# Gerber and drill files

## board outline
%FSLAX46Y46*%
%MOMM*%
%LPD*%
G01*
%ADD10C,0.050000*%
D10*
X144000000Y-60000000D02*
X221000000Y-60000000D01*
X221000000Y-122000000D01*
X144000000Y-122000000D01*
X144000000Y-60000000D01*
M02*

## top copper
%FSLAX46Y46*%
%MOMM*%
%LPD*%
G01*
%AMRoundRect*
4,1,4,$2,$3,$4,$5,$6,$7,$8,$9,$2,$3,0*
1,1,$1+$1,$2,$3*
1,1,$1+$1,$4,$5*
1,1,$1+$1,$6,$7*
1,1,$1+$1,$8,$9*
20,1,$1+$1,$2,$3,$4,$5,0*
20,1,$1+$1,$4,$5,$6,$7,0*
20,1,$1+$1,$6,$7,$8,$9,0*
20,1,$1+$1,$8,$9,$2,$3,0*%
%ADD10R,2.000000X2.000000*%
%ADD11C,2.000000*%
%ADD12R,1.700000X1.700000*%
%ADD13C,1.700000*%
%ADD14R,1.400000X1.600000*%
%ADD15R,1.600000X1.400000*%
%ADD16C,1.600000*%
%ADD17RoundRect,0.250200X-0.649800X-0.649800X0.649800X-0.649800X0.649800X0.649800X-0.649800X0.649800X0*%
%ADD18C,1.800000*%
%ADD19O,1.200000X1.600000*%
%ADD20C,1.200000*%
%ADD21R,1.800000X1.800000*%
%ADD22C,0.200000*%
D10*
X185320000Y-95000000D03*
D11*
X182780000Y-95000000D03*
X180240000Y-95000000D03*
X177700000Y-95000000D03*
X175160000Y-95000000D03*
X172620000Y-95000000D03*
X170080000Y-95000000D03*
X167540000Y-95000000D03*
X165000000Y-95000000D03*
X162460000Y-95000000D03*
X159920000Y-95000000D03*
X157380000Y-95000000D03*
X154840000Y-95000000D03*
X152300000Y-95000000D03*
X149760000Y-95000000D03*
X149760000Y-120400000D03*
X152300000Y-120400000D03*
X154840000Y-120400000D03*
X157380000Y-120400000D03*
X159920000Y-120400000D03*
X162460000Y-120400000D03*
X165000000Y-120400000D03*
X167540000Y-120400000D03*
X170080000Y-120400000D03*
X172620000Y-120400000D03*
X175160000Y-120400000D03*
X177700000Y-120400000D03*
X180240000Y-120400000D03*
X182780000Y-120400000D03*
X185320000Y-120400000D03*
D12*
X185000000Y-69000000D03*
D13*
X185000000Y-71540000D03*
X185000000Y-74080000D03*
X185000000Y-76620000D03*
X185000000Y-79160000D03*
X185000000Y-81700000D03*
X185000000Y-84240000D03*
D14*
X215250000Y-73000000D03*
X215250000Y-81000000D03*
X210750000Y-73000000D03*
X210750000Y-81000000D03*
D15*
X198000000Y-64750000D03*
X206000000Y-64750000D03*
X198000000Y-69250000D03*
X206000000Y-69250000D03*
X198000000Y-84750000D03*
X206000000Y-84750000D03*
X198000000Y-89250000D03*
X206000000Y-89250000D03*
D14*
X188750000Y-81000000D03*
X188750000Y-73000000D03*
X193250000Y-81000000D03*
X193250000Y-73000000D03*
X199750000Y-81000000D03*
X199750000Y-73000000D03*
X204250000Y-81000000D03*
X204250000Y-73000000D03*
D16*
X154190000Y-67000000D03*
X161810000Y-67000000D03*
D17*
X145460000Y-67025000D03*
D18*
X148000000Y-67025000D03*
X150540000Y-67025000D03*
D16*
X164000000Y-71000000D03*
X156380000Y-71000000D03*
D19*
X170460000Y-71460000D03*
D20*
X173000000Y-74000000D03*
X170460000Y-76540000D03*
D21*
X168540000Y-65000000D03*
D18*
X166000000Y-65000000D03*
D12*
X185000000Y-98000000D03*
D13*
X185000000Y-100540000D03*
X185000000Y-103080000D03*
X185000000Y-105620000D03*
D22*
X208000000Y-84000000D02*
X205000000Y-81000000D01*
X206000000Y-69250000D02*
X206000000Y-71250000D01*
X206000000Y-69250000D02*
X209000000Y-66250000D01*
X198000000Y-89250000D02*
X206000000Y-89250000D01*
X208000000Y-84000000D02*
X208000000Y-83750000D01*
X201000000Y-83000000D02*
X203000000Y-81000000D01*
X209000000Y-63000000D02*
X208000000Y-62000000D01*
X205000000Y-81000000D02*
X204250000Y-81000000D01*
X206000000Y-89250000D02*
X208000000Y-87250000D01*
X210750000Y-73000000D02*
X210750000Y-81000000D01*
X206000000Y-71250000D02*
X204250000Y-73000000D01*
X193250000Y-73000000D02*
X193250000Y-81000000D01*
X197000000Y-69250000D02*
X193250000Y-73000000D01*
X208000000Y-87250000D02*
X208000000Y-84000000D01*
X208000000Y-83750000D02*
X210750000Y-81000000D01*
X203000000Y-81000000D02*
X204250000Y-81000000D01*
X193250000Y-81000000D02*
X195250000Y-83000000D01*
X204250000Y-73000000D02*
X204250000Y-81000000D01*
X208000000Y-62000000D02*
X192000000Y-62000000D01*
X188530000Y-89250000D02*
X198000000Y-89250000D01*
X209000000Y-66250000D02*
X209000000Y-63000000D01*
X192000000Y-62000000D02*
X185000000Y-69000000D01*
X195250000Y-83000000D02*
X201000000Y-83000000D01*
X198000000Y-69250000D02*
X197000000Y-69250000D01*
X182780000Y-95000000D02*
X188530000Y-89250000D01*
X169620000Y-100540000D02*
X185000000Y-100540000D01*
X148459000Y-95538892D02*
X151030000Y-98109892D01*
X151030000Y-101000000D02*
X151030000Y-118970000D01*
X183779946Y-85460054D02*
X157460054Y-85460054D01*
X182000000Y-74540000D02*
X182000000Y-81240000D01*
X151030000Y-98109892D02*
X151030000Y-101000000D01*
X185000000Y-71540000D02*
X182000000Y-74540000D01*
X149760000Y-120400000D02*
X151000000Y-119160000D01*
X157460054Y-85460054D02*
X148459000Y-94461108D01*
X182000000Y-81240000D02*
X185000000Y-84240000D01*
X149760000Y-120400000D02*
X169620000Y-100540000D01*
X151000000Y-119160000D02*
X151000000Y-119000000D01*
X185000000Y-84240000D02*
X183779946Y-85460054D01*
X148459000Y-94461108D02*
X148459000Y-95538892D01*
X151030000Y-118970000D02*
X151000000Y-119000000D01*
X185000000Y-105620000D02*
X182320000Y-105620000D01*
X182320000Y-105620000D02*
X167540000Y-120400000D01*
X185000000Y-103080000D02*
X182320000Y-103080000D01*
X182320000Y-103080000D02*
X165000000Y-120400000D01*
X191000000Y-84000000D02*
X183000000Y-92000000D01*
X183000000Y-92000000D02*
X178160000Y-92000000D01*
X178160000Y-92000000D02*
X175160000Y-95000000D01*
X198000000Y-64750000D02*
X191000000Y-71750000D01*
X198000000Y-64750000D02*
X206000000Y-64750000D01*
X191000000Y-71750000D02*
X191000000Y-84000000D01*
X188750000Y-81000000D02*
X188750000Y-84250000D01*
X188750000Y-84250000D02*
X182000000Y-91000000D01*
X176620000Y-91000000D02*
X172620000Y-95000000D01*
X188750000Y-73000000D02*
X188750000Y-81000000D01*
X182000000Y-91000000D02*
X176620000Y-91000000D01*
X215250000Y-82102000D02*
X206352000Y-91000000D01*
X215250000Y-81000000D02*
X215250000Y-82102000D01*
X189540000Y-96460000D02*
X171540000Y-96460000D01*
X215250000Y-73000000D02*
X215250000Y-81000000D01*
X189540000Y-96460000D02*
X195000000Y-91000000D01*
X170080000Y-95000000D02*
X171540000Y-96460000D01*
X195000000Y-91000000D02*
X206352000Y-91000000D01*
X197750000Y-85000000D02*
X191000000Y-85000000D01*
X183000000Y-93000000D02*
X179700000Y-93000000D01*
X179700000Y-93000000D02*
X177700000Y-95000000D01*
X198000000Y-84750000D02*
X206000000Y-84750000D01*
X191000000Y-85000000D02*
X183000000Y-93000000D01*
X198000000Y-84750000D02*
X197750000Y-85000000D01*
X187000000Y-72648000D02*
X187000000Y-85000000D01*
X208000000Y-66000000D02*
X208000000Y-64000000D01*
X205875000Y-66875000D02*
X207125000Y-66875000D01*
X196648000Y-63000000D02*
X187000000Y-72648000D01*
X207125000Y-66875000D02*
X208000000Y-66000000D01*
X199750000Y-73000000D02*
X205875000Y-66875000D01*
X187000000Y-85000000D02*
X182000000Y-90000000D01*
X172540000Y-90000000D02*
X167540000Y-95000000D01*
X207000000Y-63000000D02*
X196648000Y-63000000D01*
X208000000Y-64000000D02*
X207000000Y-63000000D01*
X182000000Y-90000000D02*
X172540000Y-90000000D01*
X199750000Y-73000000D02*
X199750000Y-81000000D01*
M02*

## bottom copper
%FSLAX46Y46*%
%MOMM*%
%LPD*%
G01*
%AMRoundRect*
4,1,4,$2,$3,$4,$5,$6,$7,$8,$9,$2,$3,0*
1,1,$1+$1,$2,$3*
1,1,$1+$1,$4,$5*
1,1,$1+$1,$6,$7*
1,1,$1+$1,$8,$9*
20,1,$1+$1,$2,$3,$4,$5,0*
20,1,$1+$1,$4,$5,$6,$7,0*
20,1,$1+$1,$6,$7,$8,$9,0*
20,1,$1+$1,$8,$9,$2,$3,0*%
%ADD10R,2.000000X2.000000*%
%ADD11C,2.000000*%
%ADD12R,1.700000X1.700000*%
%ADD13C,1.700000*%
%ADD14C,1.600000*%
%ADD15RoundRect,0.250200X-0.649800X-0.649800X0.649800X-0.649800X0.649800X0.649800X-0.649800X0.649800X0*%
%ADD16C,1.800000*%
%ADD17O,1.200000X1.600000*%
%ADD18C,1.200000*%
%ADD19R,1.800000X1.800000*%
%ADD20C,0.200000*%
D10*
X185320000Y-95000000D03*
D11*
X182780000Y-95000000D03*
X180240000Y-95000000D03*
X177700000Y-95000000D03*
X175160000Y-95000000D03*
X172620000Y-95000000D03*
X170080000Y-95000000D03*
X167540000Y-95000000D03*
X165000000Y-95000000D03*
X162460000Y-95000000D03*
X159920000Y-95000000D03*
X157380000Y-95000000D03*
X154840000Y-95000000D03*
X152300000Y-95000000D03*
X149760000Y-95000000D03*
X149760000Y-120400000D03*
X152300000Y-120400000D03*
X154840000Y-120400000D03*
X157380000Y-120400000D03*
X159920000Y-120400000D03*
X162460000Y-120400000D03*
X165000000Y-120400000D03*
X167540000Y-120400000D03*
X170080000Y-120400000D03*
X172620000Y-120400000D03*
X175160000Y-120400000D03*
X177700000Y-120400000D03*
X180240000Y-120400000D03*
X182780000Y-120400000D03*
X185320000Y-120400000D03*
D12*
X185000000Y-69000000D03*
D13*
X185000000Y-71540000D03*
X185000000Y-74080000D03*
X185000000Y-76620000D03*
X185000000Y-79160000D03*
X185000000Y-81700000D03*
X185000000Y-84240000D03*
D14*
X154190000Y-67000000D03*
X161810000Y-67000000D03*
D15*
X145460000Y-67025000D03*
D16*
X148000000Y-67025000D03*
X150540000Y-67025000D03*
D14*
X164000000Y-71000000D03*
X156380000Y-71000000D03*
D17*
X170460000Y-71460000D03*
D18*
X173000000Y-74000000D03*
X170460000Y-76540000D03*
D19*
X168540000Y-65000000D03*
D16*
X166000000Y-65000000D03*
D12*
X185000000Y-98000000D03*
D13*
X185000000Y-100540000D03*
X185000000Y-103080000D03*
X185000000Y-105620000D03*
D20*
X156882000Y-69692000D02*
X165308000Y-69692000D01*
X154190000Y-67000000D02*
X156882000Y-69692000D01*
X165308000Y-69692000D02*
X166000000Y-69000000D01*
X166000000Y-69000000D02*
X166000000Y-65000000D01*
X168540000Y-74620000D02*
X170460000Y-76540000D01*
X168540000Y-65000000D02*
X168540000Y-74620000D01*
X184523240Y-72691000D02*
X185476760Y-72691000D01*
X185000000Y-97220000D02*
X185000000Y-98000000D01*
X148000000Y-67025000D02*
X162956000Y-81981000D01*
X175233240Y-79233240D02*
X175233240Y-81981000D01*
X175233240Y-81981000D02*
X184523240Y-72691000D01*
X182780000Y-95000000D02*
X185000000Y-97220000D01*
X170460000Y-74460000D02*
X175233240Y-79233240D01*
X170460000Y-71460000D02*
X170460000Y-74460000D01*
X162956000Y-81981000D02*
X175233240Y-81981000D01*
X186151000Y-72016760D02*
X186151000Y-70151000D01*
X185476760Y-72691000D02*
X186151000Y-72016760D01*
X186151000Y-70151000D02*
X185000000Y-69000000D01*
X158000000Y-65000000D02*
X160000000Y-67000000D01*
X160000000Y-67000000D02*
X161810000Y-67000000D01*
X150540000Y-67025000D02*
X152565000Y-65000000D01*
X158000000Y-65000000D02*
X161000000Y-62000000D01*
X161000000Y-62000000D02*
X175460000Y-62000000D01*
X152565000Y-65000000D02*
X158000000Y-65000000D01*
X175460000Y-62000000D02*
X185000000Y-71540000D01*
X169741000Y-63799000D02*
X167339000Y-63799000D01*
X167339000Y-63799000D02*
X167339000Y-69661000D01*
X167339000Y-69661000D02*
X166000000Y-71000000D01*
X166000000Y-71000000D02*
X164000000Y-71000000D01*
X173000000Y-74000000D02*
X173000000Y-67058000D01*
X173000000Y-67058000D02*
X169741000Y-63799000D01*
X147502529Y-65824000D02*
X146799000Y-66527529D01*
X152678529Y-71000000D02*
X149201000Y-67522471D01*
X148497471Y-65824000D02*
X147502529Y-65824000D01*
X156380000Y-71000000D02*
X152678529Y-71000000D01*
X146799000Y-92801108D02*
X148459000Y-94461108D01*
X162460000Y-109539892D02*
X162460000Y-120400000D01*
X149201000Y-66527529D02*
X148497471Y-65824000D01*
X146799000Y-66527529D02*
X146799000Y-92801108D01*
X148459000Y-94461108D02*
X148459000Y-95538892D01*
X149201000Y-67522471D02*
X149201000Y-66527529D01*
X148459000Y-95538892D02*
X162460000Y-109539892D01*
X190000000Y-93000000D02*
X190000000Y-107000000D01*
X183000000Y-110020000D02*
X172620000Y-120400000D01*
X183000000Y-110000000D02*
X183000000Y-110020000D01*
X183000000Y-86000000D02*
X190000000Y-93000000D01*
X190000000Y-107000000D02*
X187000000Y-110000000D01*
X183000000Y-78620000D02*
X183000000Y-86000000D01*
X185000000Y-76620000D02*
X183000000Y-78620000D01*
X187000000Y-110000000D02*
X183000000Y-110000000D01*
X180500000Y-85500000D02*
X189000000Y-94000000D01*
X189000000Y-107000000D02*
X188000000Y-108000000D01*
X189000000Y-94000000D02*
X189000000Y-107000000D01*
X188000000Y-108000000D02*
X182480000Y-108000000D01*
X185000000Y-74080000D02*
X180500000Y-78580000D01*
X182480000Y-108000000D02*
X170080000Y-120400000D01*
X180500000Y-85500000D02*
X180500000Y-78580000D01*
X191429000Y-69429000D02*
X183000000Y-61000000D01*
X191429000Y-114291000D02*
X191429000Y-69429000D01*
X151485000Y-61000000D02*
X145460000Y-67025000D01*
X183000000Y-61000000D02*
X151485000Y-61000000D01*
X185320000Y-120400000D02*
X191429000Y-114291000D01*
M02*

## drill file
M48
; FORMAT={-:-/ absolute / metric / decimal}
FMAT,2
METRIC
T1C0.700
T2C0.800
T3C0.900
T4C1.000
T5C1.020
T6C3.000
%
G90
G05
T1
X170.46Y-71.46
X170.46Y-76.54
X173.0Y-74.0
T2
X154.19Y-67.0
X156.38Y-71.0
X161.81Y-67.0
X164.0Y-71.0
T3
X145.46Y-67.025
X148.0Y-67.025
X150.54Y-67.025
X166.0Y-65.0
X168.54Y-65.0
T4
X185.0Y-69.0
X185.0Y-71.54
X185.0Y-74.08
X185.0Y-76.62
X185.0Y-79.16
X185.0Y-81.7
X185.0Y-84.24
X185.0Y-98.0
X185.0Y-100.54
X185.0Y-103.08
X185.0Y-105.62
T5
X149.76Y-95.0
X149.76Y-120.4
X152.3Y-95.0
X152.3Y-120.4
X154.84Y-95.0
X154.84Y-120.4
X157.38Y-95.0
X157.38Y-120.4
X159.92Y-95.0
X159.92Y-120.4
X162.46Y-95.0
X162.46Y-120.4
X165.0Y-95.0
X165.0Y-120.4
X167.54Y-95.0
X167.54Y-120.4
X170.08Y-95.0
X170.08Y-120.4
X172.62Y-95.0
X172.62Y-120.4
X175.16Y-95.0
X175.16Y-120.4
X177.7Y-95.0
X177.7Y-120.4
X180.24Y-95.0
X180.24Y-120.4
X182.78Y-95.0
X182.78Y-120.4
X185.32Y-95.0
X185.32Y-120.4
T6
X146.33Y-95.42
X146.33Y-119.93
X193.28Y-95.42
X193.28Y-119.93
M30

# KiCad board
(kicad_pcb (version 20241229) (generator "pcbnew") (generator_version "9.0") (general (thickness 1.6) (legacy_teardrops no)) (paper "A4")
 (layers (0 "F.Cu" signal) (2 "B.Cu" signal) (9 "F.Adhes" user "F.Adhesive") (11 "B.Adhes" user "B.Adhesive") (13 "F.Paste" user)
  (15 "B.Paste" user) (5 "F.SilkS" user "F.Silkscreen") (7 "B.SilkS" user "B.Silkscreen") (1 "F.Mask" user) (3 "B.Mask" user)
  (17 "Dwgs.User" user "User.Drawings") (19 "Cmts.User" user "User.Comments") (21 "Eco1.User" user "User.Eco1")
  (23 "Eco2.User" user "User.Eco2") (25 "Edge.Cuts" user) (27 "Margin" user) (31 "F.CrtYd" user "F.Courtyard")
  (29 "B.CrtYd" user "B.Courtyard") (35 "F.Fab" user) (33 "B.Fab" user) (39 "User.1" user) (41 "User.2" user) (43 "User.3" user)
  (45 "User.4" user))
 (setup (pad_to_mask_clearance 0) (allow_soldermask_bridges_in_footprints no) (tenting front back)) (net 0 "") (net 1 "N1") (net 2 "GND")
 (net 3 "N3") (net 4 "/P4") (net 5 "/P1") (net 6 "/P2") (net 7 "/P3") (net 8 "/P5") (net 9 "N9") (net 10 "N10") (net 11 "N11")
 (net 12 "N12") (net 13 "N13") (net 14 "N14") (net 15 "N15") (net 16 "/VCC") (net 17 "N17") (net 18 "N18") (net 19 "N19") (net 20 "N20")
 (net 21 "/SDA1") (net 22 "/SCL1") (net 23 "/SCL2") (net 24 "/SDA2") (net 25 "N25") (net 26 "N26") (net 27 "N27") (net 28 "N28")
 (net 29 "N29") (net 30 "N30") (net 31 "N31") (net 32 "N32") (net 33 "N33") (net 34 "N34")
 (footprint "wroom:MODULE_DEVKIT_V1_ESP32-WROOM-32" (layer "F.Cu") (at 169.805 107.7 -90)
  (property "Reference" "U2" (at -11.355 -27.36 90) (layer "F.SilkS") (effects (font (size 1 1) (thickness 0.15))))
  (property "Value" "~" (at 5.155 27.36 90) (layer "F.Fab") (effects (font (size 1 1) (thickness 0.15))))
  (pad "" np_thru_hole circle (at -12.28 -23.475 270) (size 3 3) (drill 3) (layers "*.Cu" "*.Mask"))
  (pad "" np_thru_hole circle (at -12.28 23.475 270) (size 3 3) (drill 3) (layers "*.Cu" "*.Mask"))
  (pad "" np_thru_hole circle (at 12.23 -23.475 270) (size 3 3) (drill 3) (layers "*.Cu" "*.Mask"))
  (pad "" np_thru_hole circle (at 12.23 23.475 270) (size 3 3) (drill 3) (layers "*.Cu" "*.Mask"))
  (pad "1" thru_hole rect (at -12.7 -15.515 270) (size 2 2) (drill 1.02) (layers "*.Cu" "*.Mask") (remove_unused_layers no) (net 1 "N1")
   (solder_mask_margin 0.102))
  (pad "2" thru_hole circle (at -12.7 -12.975 270) (size 2 2) (drill 1.02) (layers "*.Cu" "*.Mask") (remove_unused_layers no) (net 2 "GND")
   (solder_mask_margin 0.102))
  (pad "3" thru_hole circle (at -12.7 -10.435 270) (size 2 2) (drill 1.02) (layers "*.Cu" "*.Mask") (remove_unused_layers no) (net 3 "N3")
   (solder_mask_margin 0.102))
  (pad "4" thru_hole circle (at -12.7 -7.895 270) (size 2 2) (drill 1.02) (layers "*.Cu" "*.Mask") (remove_unused_layers no) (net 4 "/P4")
   (solder_mask_margin 0.102))
  (pad "5" thru_hole circle (at -12.7 -5.355 270) (size 2 2) (drill 1.02) (layers "*.Cu" "*.Mask") (remove_unused_layers no) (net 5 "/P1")
   (solder_mask_margin 0.102))
  (pad "6" thru_hole circle (at -12.7 -2.815 270) (size 2 2) (drill 1.02) (layers "*.Cu" "*.Mask") (remove_unused_layers no) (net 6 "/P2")
   (solder_mask_margin 0.102))
  (pad "7" thru_hole circle (at -12.7 -0.275 270) (size 2 2) (drill 1.02) (layers "*.Cu" "*.Mask") (remove_unused_layers no) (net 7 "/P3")
   (solder_mask_margin 0.102))
  (pad "8" thru_hole circle (at -12.7 2.265 270) (size 2 2) (drill 1.02) (layers "*.Cu" "*.Mask") (remove_unused_layers no) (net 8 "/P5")
   (solder_mask_margin 0.102))
  (pad "9" thru_hole circle (at -12.7 4.805 270) (size 2 2) (drill 1.02) (layers "*.Cu" "*.Mask") (remove_unused_layers no) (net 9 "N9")
   (solder_mask_margin 0.102))
  (pad "10" thru_hole circle (at -12.7 7.345 270) (size 2 2) (drill 1.02) (layers "*.Cu" "*.Mask") (remove_unused_layers no) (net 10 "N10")
   (solder_mask_margin 0.102))
  (pad "11" thru_hole circle (at -12.7 9.885 270) (size 2 2) (drill 1.02) (layers "*.Cu" "*.Mask") (remove_unused_layers no) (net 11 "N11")
   (solder_mask_margin 0.102))
  (pad "12" thru_hole circle (at -12.7 12.425 270) (size 2 2) (drill 1.02) (layers "*.Cu" "*.Mask") (remove_unused_layers no) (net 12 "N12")
   (solder_mask_margin 0.102))
  (pad "13" thru_hole circle (at -12.7 14.965 270) (size 2 2) (drill 1.02) (layers "*.Cu" "*.Mask") (remove_unused_layers no) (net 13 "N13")
   (solder_mask_margin 0.102))
  (pad "14" thru_hole circle (at -12.7 17.505 270) (size 2 2) (drill 1.02) (layers "*.Cu" "*.Mask") (remove_unused_layers no) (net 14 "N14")
   (solder_mask_margin 0.102))
  (pad "15" thru_hole circle (at -12.7 20.045 270) (size 2 2) (drill 1.02) (layers "*.Cu" "*.Mask") (remove_unused_layers no) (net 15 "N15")
   (solder_mask_margin 0.102))
  (pad "16" thru_hole circle (at 12.7 20.045 270) (size 2 2) (drill 1.02) (layers "*.Cu" "*.Mask") (remove_unused_layers no) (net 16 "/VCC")
   (solder_mask_margin 0.102))
  (pad "17" thru_hole circle (at 12.7 17.505 270) (size 2 2) (drill 1.02) (layers "*.Cu" "*.Mask") (remove_unused_layers no) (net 2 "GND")
   (solder_mask_margin 0.102))
  (pad "18" thru_hole circle (at 12.7 14.965 270) (size 2 2) (drill 1.02) (layers "*.Cu" "*.Mask") (remove_unused_layers no) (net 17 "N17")
   (solder_mask_margin 0.102))
  (pad "19" thru_hole circle (at 12.7 12.425 270) (size 2 2) (drill 1.02) (layers "*.Cu" "*.Mask") (remove_unused_layers no) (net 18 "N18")
   (solder_mask_margin 0.102))
  (pad "20" thru_hole circle (at 12.7 9.885 270) (size 2 2) (drill 1.02) (layers "*.Cu" "*.Mask") (remove_unused_layers no) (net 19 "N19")
   (solder_mask_margin 0.102))
  (pad "21" thru_hole circle (at 12.7 7.345 270) (size 2 2) (drill 1.02) (layers "*.Cu" "*.Mask") (remove_unused_layers no) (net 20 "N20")
   (solder_mask_margin 0.102))
  (pad "22" thru_hole circle (at 12.7 4.805 270) (size 2 2) (drill 1.02) (layers "*.Cu" "*.Mask") (remove_unused_layers no) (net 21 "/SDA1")
   (solder_mask_margin 0.102))
  (pad "23" thru_hole circle (at 12.7 2.265 270) (size 2 2) (drill 1.02) (layers "*.Cu" "*.Mask") (remove_unused_layers no) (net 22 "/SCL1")
   (solder_mask_margin 0.102))
  (pad "24" thru_hole circle (at 12.7 -0.275 270) (size 2 2) (drill 1.02) (layers "*.Cu" "*.Mask") (remove_unused_layers no)
   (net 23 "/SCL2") (solder_mask_margin 0.102))
  (pad "25" thru_hole circle (at 12.7 -2.815 270) (size 2 2) (drill 1.02) (layers "*.Cu" "*.Mask") (remove_unused_layers no)
   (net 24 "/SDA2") (solder_mask_margin 0.102))
  (pad "26" thru_hole circle (at 12.7 -5.355 270) (size 2 2) (drill 1.02) (layers "*.Cu" "*.Mask") (remove_unused_layers no) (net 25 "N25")
   (solder_mask_margin 0.102))
  (pad "27" thru_hole circle (at 12.7 -7.895 270) (size 2 2) (drill 1.02) (layers "*.Cu" "*.Mask") (remove_unused_layers no) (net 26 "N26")
   (solder_mask_margin 0.102))
  (pad "28" thru_hole circle (at 12.7 -10.435 270) (size 2 2) (drill 1.02) (layers "*.Cu" "*.Mask") (remove_unused_layers no) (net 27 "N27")
   (solder_mask_margin 0.102))
  (pad "29" thru_hole circle (at 12.7 -12.975 270) (size 2 2) (drill 1.02) (layers "*.Cu" "*.Mask") (remove_unused_layers no) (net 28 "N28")
   (solder_mask_margin 0.102))
  (pad "30" thru_hole circle (at 12.7 -15.515 270) (size 2 2) (drill 1.02) (layers "*.Cu" "*.Mask") (remove_unused_layers no) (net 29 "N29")
   (solder_mask_margin 0.102))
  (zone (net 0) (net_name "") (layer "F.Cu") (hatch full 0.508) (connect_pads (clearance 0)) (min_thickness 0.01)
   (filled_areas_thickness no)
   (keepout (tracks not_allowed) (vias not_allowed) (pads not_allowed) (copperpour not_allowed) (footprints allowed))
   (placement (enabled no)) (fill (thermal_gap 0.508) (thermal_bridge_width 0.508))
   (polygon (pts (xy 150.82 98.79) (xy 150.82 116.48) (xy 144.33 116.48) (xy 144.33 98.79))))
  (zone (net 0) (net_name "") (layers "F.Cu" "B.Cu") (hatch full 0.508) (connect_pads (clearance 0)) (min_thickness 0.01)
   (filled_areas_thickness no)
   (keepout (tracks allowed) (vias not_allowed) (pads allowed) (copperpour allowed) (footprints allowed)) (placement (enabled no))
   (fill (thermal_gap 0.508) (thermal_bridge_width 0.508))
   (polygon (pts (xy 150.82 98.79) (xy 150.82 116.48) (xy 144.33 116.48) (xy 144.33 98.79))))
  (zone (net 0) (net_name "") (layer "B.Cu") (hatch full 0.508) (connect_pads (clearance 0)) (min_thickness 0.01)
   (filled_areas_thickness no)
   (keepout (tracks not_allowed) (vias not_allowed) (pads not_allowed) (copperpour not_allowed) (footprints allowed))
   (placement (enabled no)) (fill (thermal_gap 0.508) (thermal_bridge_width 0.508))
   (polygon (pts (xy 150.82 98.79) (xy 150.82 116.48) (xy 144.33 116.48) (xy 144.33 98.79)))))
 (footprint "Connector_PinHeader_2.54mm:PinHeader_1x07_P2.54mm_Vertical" (layer "F.Cu") (at 185 69)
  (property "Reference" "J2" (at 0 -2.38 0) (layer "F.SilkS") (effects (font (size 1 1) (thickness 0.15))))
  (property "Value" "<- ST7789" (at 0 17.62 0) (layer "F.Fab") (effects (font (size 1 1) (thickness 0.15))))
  (pad "1" thru_hole rect (at 0 0) (size 1.7 1.7) (drill 1) (layers "*.Cu" "*.Mask") (remove_unused_layers no) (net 2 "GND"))
  (pad "2" thru_hole circle (at 0 2.54) (size 1.7 1.7) (drill 1) (layers "*.Cu" "*.Mask") (remove_unused_layers no) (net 16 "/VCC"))
  (pad "3" thru_hole circle (at 0 5.08) (size 1.7 1.7) (drill 1) (layers "*.Cu" "*.Mask") (remove_unused_layers no) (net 23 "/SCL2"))
  (pad "4" thru_hole circle (at 0 7.62) (size 1.7 1.7) (drill 1) (layers "*.Cu" "*.Mask") (remove_unused_layers no) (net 24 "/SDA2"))
  (pad "5" thru_hole circle (at 0 10.16) (size 1.7 1.7) (drill 1) (layers "*.Cu" "*.Mask") (remove_unused_layers no) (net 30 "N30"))
  (pad "6" thru_hole circle (at 0 12.7) (size 1.7 1.7) (drill 1) (layers "*.Cu" "*.Mask") (remove_unused_layers no) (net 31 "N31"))
  (pad "7" thru_hole circle (at 0 15.24) (size 1.7 1.7) (drill 1) (layers "*.Cu" "*.Mask") (remove_unused_layers no) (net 16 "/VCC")))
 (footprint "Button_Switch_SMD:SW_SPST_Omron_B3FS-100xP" (layer "F.Cu") (at 213 77 -90)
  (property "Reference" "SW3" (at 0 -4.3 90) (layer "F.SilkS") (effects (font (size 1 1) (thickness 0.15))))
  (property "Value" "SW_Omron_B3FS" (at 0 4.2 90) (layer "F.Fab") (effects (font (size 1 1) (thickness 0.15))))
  (pad "1" smd rect (at -4 -2.25 90) (size 1.6 1.4) (layers "F.Cu" "F.Mask" "F.Paste") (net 7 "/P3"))
  (pad "1" smd rect (at 4 -2.25 90) (size 1.6 1.4) (layers "F.Cu" "F.Mask" "F.Paste") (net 7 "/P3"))
  (pad "2" smd rect (at -4 2.25 90) (size 1.6 1.4) (layers "F.Cu" "F.Mask" "F.Paste") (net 2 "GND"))
  (pad "2" smd rect (at 4 2.25 90) (size 1.6 1.4) (layers "F.Cu" "F.Mask" "F.Paste") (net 2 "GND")))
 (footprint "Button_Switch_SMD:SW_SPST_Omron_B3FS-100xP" (layer "F.Cu") (at 202 67)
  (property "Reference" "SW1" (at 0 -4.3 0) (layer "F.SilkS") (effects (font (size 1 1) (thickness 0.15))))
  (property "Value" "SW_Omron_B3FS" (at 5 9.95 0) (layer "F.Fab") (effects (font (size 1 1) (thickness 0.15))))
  (pad "1" smd rect (at -4 -2.25 180) (size 1.6 1.4) (layers "F.Cu" "F.Mask" "F.Paste") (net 5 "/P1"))
  (pad "1" smd rect (at 4 -2.25 180) (size 1.6 1.4) (layers "F.Cu" "F.Mask" "F.Paste") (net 5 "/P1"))
  (pad "2" smd rect (at -4 2.25 180) (size 1.6 1.4) (layers "F.Cu" "F.Mask" "F.Paste") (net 2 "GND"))
  (pad "2" smd rect (at 4 2.25 180) (size 1.6 1.4) (layers "F.Cu" "F.Mask" "F.Paste") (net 2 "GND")))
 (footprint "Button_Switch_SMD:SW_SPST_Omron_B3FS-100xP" (layer "F.Cu") (at 202 87)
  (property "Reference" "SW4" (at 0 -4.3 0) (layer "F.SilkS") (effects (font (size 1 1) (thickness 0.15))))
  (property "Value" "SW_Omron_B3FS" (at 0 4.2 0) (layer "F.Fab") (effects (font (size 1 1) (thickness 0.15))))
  (pad "1" smd rect (at -4 -2.25 180) (size 1.6 1.4) (layers "F.Cu" "F.Mask" "F.Paste") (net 4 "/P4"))
  (pad "1" smd rect (at 4 -2.25 180) (size 1.6 1.4) (layers "F.Cu" "F.Mask" "F.Paste") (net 4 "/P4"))
  (pad "2" smd rect (at -4 2.25 180) (size 1.6 1.4) (layers "F.Cu" "F.Mask" "F.Paste") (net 2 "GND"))
  (pad "2" smd rect (at 4 2.25 180) (size 1.6 1.4) (layers "F.Cu" "F.Mask" "F.Paste") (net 2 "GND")))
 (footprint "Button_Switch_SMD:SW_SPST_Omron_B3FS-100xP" (layer "F.Cu") (at 191 77 90)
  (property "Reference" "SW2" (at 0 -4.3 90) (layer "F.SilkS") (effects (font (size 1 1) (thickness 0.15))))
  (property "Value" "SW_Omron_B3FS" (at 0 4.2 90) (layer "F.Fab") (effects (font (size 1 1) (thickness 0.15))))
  (pad "1" smd rect (at -4 -2.25 270) (size 1.6 1.4) (layers "F.Cu" "F.Mask" "F.Paste") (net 6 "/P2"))
  (pad "1" smd rect (at 4 -2.25 270) (size 1.6 1.4) (layers "F.Cu" "F.Mask" "F.Paste") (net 6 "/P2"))
  (pad "2" smd rect (at -4 2.25 270) (size 1.6 1.4) (layers "F.Cu" "F.Mask" "F.Paste") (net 2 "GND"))
  (pad "2" smd rect (at 4 2.25 270) (size 1.6 1.4) (layers "F.Cu" "F.Mask" "F.Paste") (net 2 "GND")))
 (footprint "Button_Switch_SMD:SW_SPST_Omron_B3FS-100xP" (layer "F.Cu") (at 202 77 90)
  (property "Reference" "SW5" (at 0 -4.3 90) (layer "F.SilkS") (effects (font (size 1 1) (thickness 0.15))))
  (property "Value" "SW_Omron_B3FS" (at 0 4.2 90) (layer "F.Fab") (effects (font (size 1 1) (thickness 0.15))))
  (pad "1" smd rect (at -4 -2.25 270) (size 1.6 1.4) (layers "F.Cu" "F.Mask" "F.Paste") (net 8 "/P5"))
  (pad "1" smd rect (at 4 -2.25 270) (size 1.6 1.4) (layers "F.Cu" "F.Mask" "F.Paste") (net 8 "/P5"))
  (pad "2" smd rect (at -4 2.25 270) (size 1.6 1.4) (layers "F.Cu" "F.Mask" "F.Paste") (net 2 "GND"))
  (pad "2" smd rect (at 4 2.25 270) (size 1.6 1.4) (layers "F.Cu" "F.Mask" "F.Paste") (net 2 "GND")))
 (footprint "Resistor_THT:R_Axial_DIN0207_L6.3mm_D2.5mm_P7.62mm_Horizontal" (layer "B.Cu") (at 154.19 67)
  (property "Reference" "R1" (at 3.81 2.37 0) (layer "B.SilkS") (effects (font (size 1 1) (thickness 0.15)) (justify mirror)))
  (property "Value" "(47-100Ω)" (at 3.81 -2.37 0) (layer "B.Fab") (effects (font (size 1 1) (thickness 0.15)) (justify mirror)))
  (pad "1" thru_hole circle (at 0 0) (size 1.6 1.6) (drill 0.8) (layers "*.Cu" "*.Mask") (remove_unused_layers no) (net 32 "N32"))
  (pad "2" thru_hole circle (at 7.62 0) (size 1.6 1.6) (drill 0.8) (layers "*.Cu" "*.Mask") (remove_unused_layers no) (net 16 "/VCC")))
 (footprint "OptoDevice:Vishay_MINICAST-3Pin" (layer "B.Cu") (at 145.46 67.025)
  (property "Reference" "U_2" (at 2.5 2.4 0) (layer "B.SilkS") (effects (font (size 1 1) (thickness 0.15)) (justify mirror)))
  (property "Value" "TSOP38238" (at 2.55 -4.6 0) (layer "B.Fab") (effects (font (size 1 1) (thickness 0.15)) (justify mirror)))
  (pad "1" thru_hole roundrect (at 0 0) (size 1.8 1.8) (drill 0.9) (layers "*.Cu" "*.Mask") (remove_unused_layers no)
   (roundrect_rratio 0.139) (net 29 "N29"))
  (pad "2" thru_hole circle (at 2.54 0) (size 1.8 1.8) (drill 0.9) (layers "*.Cu" "*.Mask") (remove_unused_layers no) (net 2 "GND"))
  (pad "3" thru_hole circle (at 5.08 0) (size 1.8 1.8) (drill 0.9) (layers "*.Cu" "*.Mask") (remove_unused_layers no) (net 16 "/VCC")))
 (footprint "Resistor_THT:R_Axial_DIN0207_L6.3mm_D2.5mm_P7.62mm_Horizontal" (layer "B.Cu") (at 164 71 180)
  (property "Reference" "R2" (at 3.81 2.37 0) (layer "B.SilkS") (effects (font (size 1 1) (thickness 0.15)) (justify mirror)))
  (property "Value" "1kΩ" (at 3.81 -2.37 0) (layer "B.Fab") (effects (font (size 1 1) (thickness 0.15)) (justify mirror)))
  (pad "1" thru_hole circle (at 0 0 180) (size 1.6 1.6) (drill 0.8) (layers "*.Cu" "*.Mask") (remove_unused_layers no) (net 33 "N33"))
  (pad "2" thru_hole circle (at 7.62 0 180) (size 1.6 1.6) (drill 0.8) (layers "*.Cu" "*.Mask") (remove_unused_layers no) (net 20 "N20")))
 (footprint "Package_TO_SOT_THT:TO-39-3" (layer "B.Cu") (at 170.46 71.46 -90)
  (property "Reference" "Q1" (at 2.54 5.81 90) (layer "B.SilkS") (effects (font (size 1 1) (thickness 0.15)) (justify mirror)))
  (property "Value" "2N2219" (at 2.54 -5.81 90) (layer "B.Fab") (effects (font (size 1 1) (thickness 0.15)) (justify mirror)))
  (pad "1" thru_hole oval (at 0 0 270) (size 1.6 1.2) (drill 0.7) (layers "*.Cu" "*.Mask") (remove_unused_layers no) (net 2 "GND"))
  (pad "2" thru_hole circle (at 2.54 -2.54 270) (size 1.2 1.2) (drill 0.7) (layers "*.Cu" "*.Mask") (remove_unused_layers no) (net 33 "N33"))
  (pad "3" thru_hole circle (at 5.08 0 270) (size 1.2 1.2) (drill 0.7) (layers "*.Cu" "*.Mask") (remove_unused_layers no) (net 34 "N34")))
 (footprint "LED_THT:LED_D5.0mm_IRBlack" (layer "B.Cu") (at 168.54 65 180)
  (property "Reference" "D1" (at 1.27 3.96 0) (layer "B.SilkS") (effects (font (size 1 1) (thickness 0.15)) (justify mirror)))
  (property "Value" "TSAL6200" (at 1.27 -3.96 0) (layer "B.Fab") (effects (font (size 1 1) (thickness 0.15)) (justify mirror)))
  (pad "1" thru_hole rect (at 0 0 180) (size 1.8 1.8) (drill 0.9) (layers "*.Cu" "*.Mask") (remove_unused_layers no) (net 34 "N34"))
  (pad "2" thru_hole circle (at 2.54 0 180) (size 1.8 1.8) (drill 0.9) (layers "*.Cu" "*.Mask") (remove_unused_layers no) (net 32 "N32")))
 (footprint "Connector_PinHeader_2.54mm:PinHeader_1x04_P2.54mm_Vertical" (layer "B.Cu") (at 185 98 180)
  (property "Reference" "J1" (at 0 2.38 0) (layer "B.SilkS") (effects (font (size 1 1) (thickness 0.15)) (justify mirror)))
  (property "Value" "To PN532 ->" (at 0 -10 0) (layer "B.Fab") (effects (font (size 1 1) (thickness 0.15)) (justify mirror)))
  (pad "1" thru_hole rect (at 0 0 180) (size 1.7 1.7) (drill 1) (layers "*.Cu" "*.Mask") (remove_unused_layers no) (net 2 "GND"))
  (pad "2" thru_hole circle (at 0 -2.54 180) (size 1.7 1.7) (drill 1) (layers "*.Cu" "*.Mask") (remove_unused_layers no) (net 16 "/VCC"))
  (pad "3" thru_hole circle (at 0 -5.08 180) (size 1.7 1.7) (drill 1) (layers "*.Cu" "*.Mask") (remove_unused_layers no) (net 21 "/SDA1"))
  (pad "4" thru_hole circle (at 0 -7.62 180) (size 1.7 1.7) (drill 1) (layers "*.Cu" "*.Mask") (remove_unused_layers no) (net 22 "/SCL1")))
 (gr_rect (start 144 60) (end 221 122) (stroke (width 0.05) (type default)) (fill no) (layer "Edge.Cuts"))
 (segment (start 156.882 69.692) (end 165.308 69.692) (width 0.2) (layer "B.Cu") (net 32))
 (segment (start 154.19 67) (end 156.882 69.692) (width 0.2) (layer "B.Cu") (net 32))
 (segment (start 165.308 69.692) (end 166 69) (width 0.2) (layer "B.Cu") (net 32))
 (segment (start 166 69) (end 166 65) (width 0.2) (layer "B.Cu") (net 32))
 (segment (start 168.54 74.62) (end 170.46 76.54) (width 0.2) (layer "B.Cu") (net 34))
 (segment (start 168.54 65) (end 168.54 74.62) (width 0.2) (layer "B.Cu") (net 34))
 (segment (start 208 84) (end 205 81) (width 0.2) (layer "F.Cu") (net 2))
 (segment (start 206 69.25) (end 206 71.25) (width 0.2) (layer "F.Cu") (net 2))
 (segment (start 206 69.25) (end 209 66.25) (width 0.2) (layer "F.Cu") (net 2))
 (segment (start 198 89.25) (end 206 89.25) (width 0.2) (layer "F.Cu") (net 2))
 (segment (start 208 84) (end 208 83.75) (width 0.2) (layer "F.Cu") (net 2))
 (segment (start 201 83) (end 203 81) (width 0.2) (layer "F.Cu") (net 2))
 (segment (start 209 63) (end 208 62) (width 0.2) (layer "F.Cu") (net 2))
 (segment (start 205 81) (end 204.25 81) (width 0.2) (layer "F.Cu") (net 2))
 (segment (start 206 89.25) (end 208 87.25) (width 0.2) (layer "F.Cu") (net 2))
 (segment (start 210.75 73) (end 210.75 81) (width 0.2) (layer "F.Cu") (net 2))
 (segment (start 206 71.25) (end 204.25 73) (width 0.2) (layer "F.Cu") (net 2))
 (segment (start 193.25 73) (end 193.25 81) (width 0.2) (layer "F.Cu") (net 2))
 (segment (start 197 69.25) (end 193.25 73) (width 0.2) (layer "F.Cu") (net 2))
 (segment (start 208 87.25) (end 208 84) (width 0.2) (layer "F.Cu") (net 2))
 (segment (start 208 83.75) (end 210.75 81) (width 0.2) (layer "F.Cu") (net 2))
 (segment (start 203 81) (end 204.25 81) (width 0.2) (layer "F.Cu") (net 2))
 (segment (start 193.25 81) (end 195.25 83) (width 0.2) (layer "F.Cu") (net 2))
 (segment (start 204.25 73) (end 204.25 81) (width 0.2) (layer "F.Cu") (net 2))
 (segment (start 208 62) (end 192 62) (width 0.2) (layer "F.Cu") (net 2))
 (segment (start 188.53 89.25) (end 198 89.25) (width 0.2) (layer "F.Cu") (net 2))
 (segment (start 209 66.25) (end 209 63) (width 0.2) (layer "F.Cu") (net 2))
 (segment (start 192 62) (end 185 69) (width 0.2) (layer "F.Cu") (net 2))
 (segment (start 195.25 83) (end 201 83) (width 0.2) (layer "F.Cu") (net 2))
 (segment (start 198 69.25) (end 197 69.25) (width 0.2) (layer "F.Cu") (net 2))
 (segment (start 182.78 95) (end 188.53 89.25) (width 0.2) (layer "F.Cu") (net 2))
 (segment (start 184.52324 72.691) (end 185.47676 72.691) (width 0.2) (layer "B.Cu") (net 2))
 (segment (start 185 97.22) (end 185 98) (width 0.2) (layer "B.Cu") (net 2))
 (segment (start 148 67.025) (end 162.956 81.981) (width 0.2) (layer "B.Cu") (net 2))
 (segment (start 175.23324 79.23324) (end 175.23324 81.981) (width 0.2) (layer "B.Cu") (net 2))
 (segment (start 175.23324 81.981) (end 184.52324 72.691) (width 0.2) (layer "B.Cu") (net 2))
 (segment (start 182.78 95) (end 185 97.22) (width 0.2) (layer "B.Cu") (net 2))
 (segment (start 170.46 74.46) (end 175.23324 79.23324) (width 0.2) (layer "B.Cu") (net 2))
 (segment (start 170.46 71.46) (end 170.46 74.46) (width 0.2) (layer "B.Cu") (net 2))
 (segment (start 162.956 81.981) (end 175.23324 81.981) (width 0.2) (layer "B.Cu") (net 2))
 (segment (start 186.151 72.01676) (end 186.151 70.151) (width 0.2) (layer "B.Cu") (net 2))
 (segment (start 185.47676 72.691) (end 186.151 72.01676) (width 0.2) (layer "B.Cu") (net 2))
 (segment (start 186.151 70.151) (end 185 69) (width 0.2) (layer "B.Cu") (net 2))
 (segment (start 169.62 100.54) (end 185 100.54) (width 0.2) (layer "F.Cu") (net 16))
 (segment (start 148.459 95.538892) (end 151.03 98.109892) (width 0.2) (layer "F.Cu") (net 16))
 (segment (start 151.03 101) (end 151.03 118.97) (width 0.2) (layer "F.Cu") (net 16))
 (segment (start 183.779946 85.460054) (end 157.460054 85.460054) (width 0.2) (layer "F.Cu") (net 16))
 (segment (start 182 74.54) (end 182 81.24) (width 0.2) (layer "F.Cu") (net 16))
 (segment (start 151.03 98.109892) (end 151.03 101) (width 0.2) (layer "F.Cu") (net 16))
 (segment (start 185 71.54) (end 182 74.54) (width 0.2) (layer "F.Cu") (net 16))
 (segment (start 149.76 120.4) (end 151 119.16) (width 0.2) (layer "F.Cu") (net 16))
 (segment (start 157.460054 85.460054) (end 148.459 94.461108) (width 0.2) (layer "F.Cu") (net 16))
 (segment (start 182 81.24) (end 185 84.24) (width 0.2) (layer "F.Cu") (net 16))
 (segment (start 149.76 120.4) (end 169.62 100.54) (width 0.2) (layer "F.Cu") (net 16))
 (segment (start 151 119.16) (end 151 119) (width 0.2) (layer "F.Cu") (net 16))
 (segment (start 185 84.24) (end 183.779946 85.460054) (width 0.2) (layer "F.Cu") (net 16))
 (segment (start 148.459 94.461108) (end 148.459 95.538892) (width 0.2) (layer "F.Cu") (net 16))
 (segment (start 151.03 118.97) (end 151 119) (width 0.2) (layer "F.Cu") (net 16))
 (segment (start 158 65) (end 160 67) (width 0.2) (layer "B.Cu") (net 16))
 (segment (start 160 67) (end 161.81 67) (width 0.2) (layer "B.Cu") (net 16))
 (segment (start 150.54 67.025) (end 152.565 65) (width 0.2) (layer "B.Cu") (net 16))
 (segment (start 158 65) (end 161 62) (width 0.2) (layer "B.Cu") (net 16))
 (segment (start 161 62) (end 175.46 62) (width 0.2) (layer "B.Cu") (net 16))
 (segment (start 152.565 65) (end 158 65) (width 0.2) (layer "B.Cu") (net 16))
 (segment (start 175.46 62) (end 185 71.54) (width 0.2) (layer "B.Cu") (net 16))
 (segment (start 185 105.62) (end 182.32 105.62) (width 0.2) (layer "F.Cu") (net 22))
 (segment (start 182.32 105.62) (end 167.54 120.4) (width 0.2) (layer "F.Cu") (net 22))
 (segment (start 185 103.08) (end 182.32 103.08) (width 0.2) (layer "F.Cu") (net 21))
 (segment (start 182.32 103.08) (end 165 120.4) (width 0.2) (layer "F.Cu") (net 21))
 (segment (start 169.741 63.799) (end 167.339 63.799) (width 0.2) (layer "B.Cu") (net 33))
 (segment (start 167.339 63.799) (end 167.339 69.661) (width 0.2) (layer "B.Cu") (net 33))
 (segment (start 167.339 69.661) (end 166 71) (width 0.2) (layer "B.Cu") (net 33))
 (segment (start 166 71) (end 164 71) (width 0.2) (layer "B.Cu") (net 33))
 (segment (start 173 74) (end 173 67.058) (width 0.2) (layer "B.Cu") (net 33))
 (segment (start 173 67.058) (end 169.741 63.799) (width 0.2) (layer "B.Cu") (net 33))
 (segment (start 147.502529 65.824) (end 146.799 66.527529) (width 0.2) (layer "B.Cu") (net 20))
 (segment (start 152.678529 71) (end 149.201 67.522471) (width 0.2) (layer "B.Cu") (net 20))
 (segment (start 148.497471 65.824) (end 147.502529 65.824) (width 0.2) (layer "B.Cu") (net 20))
 (segment (start 156.38 71) (end 152.678529 71) (width 0.2) (layer "B.Cu") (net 20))
 (segment (start 146.799 92.801108) (end 148.459 94.461108) (width 0.2) (layer "B.Cu") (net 20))
 (segment (start 162.46 109.539892) (end 162.46 120.4) (width 0.2) (layer "B.Cu") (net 20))
 (segment (start 149.201 66.527529) (end 148.497471 65.824) (width 0.2) (layer "B.Cu") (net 20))
 (segment (start 146.799 66.527529) (end 146.799 92.801108) (width 0.2) (layer "B.Cu") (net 20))
 (segment (start 148.459 94.461108) (end 148.459 95.538892) (width 0.2) (layer "B.Cu") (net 20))
 (segment (start 149.201 67.522471) (end 149.201 66.527529) (width 0.2) (layer "B.Cu") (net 20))
 (segment (start 148.459 95.538892) (end 162.46 109.539892) (width 0.2) (layer "B.Cu") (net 20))
 (segment (start 190 93) (end 190 107) (width 0.2) (layer "B.Cu") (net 24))
 (segment (start 183 110.02) (end 172.62 120.4) (width 0.2) (layer "B.Cu") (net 24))
 (segment (start 183 110) (end 183 110.02) (width 0.2) (layer "B.Cu") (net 24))
 (segment (start 183 86) (end 190 93) (width 0.2) (layer "B.Cu") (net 24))
 (segment (start 190 107) (end 187 110) (width 0.2) (layer "B.Cu") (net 24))
 (segment (start 183 78.62) (end 183 86) (width 0.2) (layer "B.Cu") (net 24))
 (segment (start 185 76.62) (end 183 78.62) (width 0.2) (layer "B.Cu") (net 24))
 (segment (start 187 110) (end 183 110) (width 0.2) (layer "B.Cu") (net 24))
 (segment (start 180.5 85.5) (end 189 94) (width 0.2) (layer "B.Cu") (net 23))
 (segment (start 189 107) (end 188 108) (width 0.2) (layer "B.Cu") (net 23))
 (segment (start 189 94) (end 189 107) (width 0.2) (layer "B.Cu") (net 23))
 (segment (start 188 108) (end 182.48 108) (width 0.2) (layer "B.Cu") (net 23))
 (segment (start 185 74.08) (end 180.5 78.58) (width 0.2) (layer "B.Cu") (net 23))
 (segment (start 182.48 108) (end 170.08 120.4) (width 0.2) (layer "B.Cu") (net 23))
 (segment (start 180.5 85.5) (end 180.5 78.58) (width 0.2) (layer "B.Cu") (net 23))
 (segment (start 191 84) (end 183 92) (width 0.2) (layer "F.Cu") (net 5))
 (segment (start 183 92) (end 178.16 92) (width 0.2) (layer "F.Cu") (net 5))
 (segment (start 178.16 92) (end 175.16 95) (width 0.2) (layer "F.Cu") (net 5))
 (segment (start 198 64.75) (end 191 71.75) (width 0.2) (layer "F.Cu") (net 5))
 (segment (start 198 64.75) (end 206 64.75) (width 0.2) (layer "F.Cu") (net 5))
 (segment (start 191 71.75) (end 191 84) (width 0.2) (layer "F.Cu") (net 5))
 (segment (start 188.75 81) (end 188.75 84.25) (width 0.2) (layer "F.Cu") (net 6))
 (segment (start 188.75 84.25) (end 182 91) (width 0.2) (layer "F.Cu") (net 6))
 (segment (start 176.62 91) (end 172.62 95) (width 0.2) (layer "F.Cu") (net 6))
 (segment (start 188.75 73) (end 188.75 81) (width 0.2) (layer "F.Cu") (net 6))
 (segment (start 182 91) (end 176.62 91) (width 0.2) (layer "F.Cu") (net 6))
 (segment (start 191.429 69.429) (end 183 61) (width 0.2) (layer "B.Cu") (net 29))
 (segment (start 191.429 114.291) (end 191.429 69.429) (width 0.2) (layer "B.Cu") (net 29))
 (segment (start 151.485 61) (end 145.46 67.025) (width 0.2) (layer "B.Cu") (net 29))
 (segment (start 183 61) (end 151.485 61) (width 0.2) (layer "B.Cu") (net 29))
 (segment (start 185.32 120.4) (end 191.429 114.291) (width 0.2) (layer "B.Cu") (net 29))
 (segment (start 215.25 82.102) (end 206.352 91) (width 0.2) (layer "F.Cu") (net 7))
 (segment (start 215.25 81) (end 215.25 82.102) (width 0.2) (layer "F.Cu") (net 7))
 (segment (start 189.54 96.46) (end 171.54 96.46) (width 0.2) (layer "F.Cu") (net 7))
 (segment (start 215.25 73) (end 215.25 81) (width 0.2) (layer "F.Cu") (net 7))
 (segment (start 189.54 96.46) (end 195 91) (width 0.2) (layer "F.Cu") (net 7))
 (segment (start 170.08 95) (end 171.54 96.46) (width 0.2) (layer "F.Cu") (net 7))
 (segment (start 195 91) (end 206.352 91) (width 0.2) (layer "F.Cu") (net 7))
 (segment (start 197.75 85) (end 191 85) (width 0.2) (layer "F.Cu") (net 4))
 (segment (start 183 93) (end 179.7 93) (width 0.2) (layer "F.Cu") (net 4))
 (segment (start 179.7 93) (end 177.7 95) (width 0.2) (layer "F.Cu") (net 4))
 (segment (start 198 84.75) (end 206 84.75) (width 0.2) (layer "F.Cu") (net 4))
 (segment (start 191 85) (end 183 93) (width 0.2) (layer "F.Cu") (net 4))
 (segment (start 198 84.75) (end 197.75 85) (width 0.2) (layer "F.Cu") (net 4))
 (segment (start 187 72.648) (end 187 85) (width 0.2) (layer "F.Cu") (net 8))
 (segment (start 208 66) (end 208 64) (width 0.2) (layer "F.Cu") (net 8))
 (segment (start 205.875 66.875) (end 207.125 66.875) (width 0.2) (layer "F.Cu") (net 8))
 (segment (start 196.648 63) (end 187 72.648) (width 0.2) (layer "F.Cu") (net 8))
 (segment (start 207.125 66.875) (end 208 66) (width 0.2) (layer "F.Cu") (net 8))
 (segment (start 199.75 73) (end 205.875 66.875) (width 0.2) (layer "F.Cu") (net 8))
 (segment (start 187 85) (end 182 90) (width 0.2) (layer "F.Cu") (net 8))
 (segment (start 172.54 90) (end 167.54 95) (width 0.2) (layer "F.Cu") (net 8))
 (segment (start 207 63) (end 196.648 63) (width 0.2) (layer "F.Cu") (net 8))
 (segment (start 208 64) (end 207 63) (width 0.2) (layer "F.Cu") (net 8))
 (segment (start 182 90) (end 172.54 90) (width 0.2) (layer "F.Cu") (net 8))
 (segment (start 199.75 73) (end 199.75 81) (width 0.2) (layer "F.Cu") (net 8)))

